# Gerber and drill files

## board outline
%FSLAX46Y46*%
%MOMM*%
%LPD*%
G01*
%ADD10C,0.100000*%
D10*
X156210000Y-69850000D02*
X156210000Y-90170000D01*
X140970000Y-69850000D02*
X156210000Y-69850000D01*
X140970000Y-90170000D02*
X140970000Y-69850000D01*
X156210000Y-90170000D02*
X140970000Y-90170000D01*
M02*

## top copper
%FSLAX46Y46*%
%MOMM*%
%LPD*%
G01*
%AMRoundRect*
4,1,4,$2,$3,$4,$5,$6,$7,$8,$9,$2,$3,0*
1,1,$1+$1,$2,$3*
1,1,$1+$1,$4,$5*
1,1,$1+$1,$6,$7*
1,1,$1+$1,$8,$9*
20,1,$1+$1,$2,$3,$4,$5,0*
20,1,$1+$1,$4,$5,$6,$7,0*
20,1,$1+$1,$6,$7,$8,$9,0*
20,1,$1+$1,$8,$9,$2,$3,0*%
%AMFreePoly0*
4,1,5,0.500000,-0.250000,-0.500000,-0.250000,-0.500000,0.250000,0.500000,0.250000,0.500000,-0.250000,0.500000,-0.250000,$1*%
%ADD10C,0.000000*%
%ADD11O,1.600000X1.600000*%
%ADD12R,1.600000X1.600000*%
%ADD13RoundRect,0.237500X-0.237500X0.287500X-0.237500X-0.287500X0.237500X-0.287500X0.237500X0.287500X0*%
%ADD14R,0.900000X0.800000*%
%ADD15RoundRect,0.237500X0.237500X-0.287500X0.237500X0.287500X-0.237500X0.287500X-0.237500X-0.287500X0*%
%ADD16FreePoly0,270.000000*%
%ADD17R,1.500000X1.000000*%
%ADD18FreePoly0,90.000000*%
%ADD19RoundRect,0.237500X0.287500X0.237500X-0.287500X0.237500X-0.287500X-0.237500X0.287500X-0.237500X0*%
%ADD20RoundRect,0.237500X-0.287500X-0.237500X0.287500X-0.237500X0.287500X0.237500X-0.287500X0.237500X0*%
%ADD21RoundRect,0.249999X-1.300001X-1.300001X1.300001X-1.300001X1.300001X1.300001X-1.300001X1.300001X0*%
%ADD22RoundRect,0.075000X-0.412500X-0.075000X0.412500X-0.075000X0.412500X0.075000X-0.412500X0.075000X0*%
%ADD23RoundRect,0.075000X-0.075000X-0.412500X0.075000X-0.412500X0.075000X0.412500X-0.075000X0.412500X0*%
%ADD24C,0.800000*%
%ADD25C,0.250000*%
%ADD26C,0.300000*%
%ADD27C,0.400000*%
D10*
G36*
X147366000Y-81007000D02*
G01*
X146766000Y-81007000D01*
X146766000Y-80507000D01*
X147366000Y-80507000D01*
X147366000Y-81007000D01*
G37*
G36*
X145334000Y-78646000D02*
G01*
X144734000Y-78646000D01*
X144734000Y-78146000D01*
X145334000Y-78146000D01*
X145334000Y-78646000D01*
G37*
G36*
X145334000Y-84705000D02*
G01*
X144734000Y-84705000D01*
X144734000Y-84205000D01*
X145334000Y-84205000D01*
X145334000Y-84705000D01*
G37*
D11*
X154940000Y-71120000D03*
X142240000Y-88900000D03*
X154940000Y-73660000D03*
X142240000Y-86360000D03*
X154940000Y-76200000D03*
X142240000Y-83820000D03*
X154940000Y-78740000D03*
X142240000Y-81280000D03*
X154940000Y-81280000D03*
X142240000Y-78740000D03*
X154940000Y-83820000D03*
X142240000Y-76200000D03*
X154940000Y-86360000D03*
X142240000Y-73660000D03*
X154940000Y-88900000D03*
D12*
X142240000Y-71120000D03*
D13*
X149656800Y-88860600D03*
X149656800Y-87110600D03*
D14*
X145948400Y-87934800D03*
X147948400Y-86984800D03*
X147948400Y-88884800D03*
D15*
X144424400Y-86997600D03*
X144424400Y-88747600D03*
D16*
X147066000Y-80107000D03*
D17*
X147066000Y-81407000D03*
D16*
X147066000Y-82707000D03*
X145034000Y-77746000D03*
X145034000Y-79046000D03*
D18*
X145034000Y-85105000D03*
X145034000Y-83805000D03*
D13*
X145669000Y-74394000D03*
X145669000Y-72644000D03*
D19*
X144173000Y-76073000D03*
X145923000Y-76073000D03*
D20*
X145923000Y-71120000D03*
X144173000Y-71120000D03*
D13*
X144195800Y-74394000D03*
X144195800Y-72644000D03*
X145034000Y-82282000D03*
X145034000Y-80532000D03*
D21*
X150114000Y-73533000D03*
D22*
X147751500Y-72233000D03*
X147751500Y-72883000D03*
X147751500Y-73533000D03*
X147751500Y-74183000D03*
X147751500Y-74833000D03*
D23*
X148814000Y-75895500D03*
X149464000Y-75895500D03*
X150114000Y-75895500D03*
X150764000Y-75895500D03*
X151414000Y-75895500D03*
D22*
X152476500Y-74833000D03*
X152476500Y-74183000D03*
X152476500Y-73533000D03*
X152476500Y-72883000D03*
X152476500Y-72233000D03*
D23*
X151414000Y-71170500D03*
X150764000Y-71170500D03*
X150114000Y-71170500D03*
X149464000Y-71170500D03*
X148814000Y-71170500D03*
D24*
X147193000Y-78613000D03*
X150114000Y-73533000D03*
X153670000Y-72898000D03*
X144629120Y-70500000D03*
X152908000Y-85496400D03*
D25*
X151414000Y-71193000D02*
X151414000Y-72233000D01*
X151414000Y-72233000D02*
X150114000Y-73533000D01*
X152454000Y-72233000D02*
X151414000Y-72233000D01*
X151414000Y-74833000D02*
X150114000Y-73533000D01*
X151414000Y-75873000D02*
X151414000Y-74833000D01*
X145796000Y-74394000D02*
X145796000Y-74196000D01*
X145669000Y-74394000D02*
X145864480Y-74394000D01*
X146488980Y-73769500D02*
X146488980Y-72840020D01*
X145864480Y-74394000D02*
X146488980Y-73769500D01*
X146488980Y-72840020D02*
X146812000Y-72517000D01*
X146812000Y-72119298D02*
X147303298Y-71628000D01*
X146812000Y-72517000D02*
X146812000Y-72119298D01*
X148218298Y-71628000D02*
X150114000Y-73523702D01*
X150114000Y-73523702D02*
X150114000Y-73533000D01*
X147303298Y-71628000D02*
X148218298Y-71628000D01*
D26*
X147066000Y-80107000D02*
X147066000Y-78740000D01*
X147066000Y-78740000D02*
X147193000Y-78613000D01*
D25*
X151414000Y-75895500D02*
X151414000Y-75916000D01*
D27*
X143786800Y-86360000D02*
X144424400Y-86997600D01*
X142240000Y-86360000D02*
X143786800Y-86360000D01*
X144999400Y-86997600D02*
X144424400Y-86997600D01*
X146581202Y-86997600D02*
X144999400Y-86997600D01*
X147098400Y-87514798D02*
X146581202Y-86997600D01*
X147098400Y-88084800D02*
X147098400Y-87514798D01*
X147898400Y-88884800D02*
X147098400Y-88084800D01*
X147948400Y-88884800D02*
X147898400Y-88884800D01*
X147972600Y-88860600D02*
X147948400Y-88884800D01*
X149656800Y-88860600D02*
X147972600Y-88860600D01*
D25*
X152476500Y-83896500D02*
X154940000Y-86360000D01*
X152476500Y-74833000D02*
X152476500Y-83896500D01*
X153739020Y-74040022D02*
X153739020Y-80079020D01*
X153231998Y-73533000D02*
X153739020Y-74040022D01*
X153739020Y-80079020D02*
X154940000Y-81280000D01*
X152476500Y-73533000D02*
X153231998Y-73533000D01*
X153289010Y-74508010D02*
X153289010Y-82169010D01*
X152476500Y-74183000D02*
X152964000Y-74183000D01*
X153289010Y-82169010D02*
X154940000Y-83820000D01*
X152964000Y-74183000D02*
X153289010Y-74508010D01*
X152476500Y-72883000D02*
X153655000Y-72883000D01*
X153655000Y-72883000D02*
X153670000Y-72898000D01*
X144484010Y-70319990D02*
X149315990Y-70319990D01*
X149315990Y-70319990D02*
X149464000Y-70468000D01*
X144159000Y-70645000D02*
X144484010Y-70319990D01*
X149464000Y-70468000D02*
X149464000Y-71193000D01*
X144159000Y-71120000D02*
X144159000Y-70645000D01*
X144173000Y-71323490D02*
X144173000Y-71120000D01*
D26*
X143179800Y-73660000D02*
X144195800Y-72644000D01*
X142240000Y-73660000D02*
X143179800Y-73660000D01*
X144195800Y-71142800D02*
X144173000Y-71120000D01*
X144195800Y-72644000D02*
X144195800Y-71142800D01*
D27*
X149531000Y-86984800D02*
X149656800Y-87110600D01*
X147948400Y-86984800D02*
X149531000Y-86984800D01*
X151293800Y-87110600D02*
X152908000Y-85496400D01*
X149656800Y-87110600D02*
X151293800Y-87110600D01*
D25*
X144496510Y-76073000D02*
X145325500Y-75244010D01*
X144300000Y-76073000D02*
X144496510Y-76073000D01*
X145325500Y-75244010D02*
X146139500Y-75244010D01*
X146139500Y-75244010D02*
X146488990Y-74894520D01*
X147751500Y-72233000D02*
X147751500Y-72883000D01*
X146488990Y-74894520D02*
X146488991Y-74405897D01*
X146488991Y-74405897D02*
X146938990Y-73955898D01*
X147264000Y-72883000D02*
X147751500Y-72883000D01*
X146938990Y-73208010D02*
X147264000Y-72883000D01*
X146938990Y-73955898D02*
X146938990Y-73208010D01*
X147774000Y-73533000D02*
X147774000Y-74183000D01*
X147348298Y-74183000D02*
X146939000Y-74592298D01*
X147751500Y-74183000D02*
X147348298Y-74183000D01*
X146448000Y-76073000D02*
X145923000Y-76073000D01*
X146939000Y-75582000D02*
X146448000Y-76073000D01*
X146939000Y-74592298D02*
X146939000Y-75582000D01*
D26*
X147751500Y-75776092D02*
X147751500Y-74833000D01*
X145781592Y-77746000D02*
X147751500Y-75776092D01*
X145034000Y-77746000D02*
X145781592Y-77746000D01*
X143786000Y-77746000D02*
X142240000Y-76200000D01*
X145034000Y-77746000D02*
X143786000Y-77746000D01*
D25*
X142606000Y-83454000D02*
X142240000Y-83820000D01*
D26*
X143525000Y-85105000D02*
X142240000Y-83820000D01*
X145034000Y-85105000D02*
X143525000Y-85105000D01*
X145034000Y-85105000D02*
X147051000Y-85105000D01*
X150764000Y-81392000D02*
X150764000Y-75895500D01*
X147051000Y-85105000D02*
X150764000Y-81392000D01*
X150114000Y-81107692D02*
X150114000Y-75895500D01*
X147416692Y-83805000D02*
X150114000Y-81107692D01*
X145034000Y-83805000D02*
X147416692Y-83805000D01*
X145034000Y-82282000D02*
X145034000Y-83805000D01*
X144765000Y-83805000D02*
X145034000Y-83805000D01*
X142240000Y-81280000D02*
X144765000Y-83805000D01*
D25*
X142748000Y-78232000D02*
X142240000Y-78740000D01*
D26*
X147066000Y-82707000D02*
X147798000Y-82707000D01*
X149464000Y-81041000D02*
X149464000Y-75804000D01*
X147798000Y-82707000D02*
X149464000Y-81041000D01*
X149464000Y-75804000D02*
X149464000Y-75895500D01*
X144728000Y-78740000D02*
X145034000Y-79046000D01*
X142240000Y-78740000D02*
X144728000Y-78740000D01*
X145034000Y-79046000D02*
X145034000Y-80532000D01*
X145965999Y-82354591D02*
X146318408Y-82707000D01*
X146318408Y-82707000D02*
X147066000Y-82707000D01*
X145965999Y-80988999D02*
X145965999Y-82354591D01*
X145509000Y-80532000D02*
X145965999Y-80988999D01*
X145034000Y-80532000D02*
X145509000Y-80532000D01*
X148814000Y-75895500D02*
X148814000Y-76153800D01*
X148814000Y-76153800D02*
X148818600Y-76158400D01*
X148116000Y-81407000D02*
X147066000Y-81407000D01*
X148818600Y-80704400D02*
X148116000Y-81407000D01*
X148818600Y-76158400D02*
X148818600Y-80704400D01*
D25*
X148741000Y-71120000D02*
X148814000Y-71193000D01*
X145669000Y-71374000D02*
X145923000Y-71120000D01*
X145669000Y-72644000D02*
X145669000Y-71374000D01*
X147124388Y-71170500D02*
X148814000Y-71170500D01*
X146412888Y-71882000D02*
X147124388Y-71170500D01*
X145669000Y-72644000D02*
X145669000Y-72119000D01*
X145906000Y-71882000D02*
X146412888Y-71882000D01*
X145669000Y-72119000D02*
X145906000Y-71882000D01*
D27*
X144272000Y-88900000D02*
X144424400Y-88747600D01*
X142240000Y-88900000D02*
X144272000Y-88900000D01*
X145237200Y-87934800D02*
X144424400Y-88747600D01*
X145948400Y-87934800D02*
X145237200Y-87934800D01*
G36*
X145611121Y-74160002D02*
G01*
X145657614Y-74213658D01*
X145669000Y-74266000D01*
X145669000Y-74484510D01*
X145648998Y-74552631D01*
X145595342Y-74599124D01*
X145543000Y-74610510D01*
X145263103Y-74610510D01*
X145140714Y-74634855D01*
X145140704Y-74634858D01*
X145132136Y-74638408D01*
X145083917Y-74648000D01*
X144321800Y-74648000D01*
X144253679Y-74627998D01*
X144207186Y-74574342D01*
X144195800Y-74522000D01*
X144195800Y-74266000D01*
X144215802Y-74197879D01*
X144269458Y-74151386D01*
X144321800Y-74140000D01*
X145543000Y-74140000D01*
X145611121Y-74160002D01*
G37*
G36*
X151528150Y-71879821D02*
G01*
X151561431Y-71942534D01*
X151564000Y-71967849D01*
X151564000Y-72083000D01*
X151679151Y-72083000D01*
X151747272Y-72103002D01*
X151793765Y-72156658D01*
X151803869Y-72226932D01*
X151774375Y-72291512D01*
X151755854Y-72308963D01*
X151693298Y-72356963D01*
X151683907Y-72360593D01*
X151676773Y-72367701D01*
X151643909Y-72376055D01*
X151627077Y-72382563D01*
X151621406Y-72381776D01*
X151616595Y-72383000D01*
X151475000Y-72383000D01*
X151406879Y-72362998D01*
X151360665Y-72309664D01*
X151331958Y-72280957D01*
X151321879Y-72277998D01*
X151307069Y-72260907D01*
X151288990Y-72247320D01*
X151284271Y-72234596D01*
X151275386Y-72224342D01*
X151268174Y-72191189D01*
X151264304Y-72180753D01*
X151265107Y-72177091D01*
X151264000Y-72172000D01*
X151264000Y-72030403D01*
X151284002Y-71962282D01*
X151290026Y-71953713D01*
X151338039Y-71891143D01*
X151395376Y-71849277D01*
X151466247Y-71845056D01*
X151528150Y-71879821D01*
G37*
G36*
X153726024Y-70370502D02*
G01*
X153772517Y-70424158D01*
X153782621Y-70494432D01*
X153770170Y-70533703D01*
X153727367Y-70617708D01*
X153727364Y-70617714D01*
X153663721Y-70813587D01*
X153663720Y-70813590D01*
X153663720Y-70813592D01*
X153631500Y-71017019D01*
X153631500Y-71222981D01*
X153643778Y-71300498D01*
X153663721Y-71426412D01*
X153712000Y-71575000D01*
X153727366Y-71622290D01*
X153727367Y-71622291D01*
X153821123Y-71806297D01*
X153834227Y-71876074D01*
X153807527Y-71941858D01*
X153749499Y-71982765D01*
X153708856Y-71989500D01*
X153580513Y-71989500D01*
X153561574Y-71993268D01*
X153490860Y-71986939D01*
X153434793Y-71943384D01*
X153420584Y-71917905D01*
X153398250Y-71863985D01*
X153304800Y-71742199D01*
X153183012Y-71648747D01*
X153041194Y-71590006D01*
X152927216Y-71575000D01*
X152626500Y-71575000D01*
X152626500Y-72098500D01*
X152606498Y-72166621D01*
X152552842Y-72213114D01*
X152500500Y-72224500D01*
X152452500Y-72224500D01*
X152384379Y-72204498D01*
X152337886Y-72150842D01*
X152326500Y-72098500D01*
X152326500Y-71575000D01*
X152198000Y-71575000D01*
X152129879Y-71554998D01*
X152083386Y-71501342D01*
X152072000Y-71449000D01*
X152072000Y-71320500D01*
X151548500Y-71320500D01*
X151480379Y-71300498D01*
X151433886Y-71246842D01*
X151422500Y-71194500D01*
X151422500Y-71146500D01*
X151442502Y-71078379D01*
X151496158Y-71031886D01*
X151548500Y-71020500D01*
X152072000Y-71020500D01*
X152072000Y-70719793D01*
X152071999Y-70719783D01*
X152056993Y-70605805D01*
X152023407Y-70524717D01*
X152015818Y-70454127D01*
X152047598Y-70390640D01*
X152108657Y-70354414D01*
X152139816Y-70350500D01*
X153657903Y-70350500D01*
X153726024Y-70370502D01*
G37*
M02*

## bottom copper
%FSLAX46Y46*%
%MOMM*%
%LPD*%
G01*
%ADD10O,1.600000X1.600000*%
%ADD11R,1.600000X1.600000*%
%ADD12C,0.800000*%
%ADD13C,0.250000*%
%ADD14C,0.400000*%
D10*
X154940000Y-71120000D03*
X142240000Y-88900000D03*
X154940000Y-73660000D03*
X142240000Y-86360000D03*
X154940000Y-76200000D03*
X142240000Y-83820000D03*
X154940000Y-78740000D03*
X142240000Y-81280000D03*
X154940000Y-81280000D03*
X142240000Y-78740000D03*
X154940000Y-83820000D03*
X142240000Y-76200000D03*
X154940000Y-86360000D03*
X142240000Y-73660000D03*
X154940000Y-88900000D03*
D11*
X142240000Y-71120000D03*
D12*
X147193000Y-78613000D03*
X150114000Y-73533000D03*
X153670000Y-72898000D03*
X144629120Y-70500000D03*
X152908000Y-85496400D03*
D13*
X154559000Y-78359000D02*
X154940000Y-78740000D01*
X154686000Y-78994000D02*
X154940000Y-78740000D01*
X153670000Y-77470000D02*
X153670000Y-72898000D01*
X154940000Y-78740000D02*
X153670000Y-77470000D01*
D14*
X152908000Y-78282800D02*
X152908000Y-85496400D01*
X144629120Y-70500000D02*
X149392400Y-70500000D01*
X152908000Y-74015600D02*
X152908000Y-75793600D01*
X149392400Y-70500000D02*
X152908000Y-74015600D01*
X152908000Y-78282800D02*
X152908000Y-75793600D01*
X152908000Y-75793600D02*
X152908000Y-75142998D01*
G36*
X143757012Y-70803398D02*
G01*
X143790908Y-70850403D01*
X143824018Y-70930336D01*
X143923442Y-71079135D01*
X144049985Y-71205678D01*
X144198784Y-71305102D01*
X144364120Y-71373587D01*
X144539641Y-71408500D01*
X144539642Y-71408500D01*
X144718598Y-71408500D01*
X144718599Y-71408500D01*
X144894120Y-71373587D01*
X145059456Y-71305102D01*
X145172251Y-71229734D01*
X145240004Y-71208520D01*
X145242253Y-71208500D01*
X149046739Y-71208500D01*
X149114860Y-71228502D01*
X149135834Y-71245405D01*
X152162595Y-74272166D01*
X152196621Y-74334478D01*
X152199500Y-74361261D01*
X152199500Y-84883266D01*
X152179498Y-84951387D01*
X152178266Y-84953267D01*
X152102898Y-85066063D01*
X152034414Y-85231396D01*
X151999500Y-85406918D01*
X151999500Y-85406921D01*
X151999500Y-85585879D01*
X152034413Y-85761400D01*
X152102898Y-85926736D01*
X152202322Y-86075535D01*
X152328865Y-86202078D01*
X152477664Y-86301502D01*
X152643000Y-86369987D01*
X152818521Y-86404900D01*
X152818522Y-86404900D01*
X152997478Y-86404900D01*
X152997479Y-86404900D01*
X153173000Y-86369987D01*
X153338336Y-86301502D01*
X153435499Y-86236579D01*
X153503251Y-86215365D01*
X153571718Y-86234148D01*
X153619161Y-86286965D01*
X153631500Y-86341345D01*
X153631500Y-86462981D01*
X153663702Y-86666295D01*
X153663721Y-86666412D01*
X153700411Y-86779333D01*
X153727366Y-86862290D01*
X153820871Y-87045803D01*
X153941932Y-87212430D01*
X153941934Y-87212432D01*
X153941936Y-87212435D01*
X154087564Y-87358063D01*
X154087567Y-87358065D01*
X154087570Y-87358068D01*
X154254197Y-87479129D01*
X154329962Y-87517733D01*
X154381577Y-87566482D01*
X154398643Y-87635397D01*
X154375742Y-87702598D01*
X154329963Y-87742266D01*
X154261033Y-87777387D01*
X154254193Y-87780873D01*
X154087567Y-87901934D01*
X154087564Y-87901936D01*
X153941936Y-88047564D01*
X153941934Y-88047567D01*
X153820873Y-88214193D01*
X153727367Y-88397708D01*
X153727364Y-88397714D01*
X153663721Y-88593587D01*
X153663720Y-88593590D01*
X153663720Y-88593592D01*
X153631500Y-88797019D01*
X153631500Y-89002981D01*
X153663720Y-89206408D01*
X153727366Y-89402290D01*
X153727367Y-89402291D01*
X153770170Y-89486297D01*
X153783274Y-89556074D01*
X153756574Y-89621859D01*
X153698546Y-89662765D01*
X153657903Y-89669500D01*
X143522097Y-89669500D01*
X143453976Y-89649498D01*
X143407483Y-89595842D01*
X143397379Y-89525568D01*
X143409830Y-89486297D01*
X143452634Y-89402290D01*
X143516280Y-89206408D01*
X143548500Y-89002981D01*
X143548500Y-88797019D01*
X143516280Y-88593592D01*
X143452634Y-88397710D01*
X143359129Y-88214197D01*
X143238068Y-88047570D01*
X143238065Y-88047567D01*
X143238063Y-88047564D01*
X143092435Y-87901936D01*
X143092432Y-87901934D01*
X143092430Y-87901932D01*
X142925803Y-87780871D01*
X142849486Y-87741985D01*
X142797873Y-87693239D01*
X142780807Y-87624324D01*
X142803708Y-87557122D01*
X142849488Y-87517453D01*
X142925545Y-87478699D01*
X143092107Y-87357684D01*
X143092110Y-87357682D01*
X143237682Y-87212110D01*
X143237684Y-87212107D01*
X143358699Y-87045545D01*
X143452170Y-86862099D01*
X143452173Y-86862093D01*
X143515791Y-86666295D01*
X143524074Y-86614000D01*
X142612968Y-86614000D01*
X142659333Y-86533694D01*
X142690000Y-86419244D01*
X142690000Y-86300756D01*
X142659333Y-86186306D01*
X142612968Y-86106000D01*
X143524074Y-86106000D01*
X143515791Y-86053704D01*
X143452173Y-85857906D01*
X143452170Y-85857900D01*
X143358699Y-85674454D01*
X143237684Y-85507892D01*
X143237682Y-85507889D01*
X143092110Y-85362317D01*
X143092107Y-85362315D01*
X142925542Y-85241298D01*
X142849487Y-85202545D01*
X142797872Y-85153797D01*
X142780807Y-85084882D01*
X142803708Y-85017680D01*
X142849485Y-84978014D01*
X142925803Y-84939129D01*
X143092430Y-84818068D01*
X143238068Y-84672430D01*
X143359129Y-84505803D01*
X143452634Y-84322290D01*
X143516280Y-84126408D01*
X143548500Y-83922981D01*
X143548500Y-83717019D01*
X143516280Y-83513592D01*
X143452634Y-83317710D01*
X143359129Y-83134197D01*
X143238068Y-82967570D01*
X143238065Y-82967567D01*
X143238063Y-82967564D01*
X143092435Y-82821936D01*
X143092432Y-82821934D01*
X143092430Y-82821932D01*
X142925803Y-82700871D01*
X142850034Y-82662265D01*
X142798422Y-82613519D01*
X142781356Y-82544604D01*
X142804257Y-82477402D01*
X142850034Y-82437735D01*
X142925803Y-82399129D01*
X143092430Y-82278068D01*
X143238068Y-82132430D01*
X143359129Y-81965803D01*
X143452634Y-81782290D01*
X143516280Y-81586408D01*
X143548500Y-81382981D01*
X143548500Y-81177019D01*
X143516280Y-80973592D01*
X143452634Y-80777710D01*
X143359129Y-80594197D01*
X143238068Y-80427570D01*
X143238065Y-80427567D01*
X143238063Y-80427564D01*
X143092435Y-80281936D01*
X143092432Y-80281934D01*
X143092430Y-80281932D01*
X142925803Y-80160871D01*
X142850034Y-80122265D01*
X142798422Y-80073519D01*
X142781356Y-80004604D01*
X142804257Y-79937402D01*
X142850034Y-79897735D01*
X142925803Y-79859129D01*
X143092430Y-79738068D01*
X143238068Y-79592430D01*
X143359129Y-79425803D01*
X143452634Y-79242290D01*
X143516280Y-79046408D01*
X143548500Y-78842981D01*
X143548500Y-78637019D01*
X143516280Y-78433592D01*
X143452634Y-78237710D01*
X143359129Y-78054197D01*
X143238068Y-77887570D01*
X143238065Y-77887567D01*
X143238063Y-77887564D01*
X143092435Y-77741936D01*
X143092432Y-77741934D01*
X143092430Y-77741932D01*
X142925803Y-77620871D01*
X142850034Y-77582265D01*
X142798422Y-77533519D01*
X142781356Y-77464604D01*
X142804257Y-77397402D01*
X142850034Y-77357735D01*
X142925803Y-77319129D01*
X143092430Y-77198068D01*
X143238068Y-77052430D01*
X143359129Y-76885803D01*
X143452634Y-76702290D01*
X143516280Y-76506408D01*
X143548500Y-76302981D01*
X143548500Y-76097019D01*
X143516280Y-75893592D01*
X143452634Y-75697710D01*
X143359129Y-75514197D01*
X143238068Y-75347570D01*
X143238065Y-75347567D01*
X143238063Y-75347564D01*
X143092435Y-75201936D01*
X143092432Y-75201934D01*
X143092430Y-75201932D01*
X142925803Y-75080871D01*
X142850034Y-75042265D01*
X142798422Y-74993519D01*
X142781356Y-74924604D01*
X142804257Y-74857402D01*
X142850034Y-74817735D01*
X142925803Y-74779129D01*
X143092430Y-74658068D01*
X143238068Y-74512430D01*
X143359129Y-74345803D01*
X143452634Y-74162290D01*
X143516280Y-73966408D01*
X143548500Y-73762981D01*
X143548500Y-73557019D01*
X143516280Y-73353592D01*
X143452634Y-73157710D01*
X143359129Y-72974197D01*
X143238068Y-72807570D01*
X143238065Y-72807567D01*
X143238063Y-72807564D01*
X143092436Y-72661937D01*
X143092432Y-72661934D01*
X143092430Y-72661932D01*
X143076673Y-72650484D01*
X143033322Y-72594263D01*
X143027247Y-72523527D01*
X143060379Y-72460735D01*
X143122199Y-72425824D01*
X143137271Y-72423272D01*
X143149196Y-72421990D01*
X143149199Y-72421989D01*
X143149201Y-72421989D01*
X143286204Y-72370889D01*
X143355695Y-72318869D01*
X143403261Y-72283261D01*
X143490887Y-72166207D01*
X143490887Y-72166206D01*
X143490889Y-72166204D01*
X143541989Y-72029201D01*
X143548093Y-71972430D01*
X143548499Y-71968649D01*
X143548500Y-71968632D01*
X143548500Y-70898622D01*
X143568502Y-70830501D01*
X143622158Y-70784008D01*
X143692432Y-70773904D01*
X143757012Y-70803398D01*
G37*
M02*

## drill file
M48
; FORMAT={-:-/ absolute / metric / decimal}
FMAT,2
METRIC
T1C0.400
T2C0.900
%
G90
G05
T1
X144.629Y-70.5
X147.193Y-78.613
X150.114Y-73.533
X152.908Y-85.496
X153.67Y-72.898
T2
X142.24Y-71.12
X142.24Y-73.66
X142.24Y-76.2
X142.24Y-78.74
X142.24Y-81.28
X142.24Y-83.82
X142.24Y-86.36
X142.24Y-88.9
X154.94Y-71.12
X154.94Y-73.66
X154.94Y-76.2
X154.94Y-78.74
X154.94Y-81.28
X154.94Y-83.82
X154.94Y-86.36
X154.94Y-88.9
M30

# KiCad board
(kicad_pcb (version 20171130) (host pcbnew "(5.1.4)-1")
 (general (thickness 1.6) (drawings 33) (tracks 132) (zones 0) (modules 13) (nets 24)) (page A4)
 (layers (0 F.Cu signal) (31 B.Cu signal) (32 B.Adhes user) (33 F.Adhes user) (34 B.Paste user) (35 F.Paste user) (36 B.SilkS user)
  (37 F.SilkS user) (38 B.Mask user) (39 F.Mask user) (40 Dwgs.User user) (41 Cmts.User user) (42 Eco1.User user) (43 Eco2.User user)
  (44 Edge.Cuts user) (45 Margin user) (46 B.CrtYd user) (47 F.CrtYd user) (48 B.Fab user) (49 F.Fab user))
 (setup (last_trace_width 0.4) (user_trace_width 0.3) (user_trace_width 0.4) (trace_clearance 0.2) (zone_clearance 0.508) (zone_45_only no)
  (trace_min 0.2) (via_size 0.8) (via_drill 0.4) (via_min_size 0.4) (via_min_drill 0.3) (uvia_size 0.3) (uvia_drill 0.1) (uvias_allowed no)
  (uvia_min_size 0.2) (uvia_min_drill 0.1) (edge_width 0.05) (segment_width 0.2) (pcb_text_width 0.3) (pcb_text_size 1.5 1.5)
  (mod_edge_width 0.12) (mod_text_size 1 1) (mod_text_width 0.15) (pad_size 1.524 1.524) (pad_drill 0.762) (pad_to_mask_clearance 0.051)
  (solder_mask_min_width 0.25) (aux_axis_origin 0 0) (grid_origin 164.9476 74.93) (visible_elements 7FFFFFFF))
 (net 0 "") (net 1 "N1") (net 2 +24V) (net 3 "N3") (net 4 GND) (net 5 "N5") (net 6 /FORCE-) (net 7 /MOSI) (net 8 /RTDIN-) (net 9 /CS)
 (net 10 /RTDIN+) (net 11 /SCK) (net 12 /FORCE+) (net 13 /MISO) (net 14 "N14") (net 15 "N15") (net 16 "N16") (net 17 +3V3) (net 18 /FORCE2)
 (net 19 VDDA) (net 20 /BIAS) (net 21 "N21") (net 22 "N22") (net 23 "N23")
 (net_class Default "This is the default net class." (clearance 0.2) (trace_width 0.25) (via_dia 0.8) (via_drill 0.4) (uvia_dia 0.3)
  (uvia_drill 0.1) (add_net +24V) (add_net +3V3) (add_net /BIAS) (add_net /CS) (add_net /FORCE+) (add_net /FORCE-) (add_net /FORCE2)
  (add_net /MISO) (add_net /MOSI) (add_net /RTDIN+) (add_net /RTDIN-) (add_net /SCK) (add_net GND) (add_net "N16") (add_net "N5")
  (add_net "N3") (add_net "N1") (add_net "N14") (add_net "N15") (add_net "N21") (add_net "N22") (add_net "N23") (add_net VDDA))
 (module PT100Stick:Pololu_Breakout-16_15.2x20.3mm (layer F.Cu) (at 142.24 71.12)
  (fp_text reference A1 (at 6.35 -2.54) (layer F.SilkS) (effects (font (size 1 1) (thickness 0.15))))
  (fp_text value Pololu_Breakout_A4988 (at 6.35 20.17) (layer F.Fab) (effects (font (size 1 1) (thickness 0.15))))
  (pad 16 thru_hole oval (at 12.7 0) (size 1.6 1.6) (drill 0.9) (layers *.Cu *.Mask) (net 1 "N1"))
  (pad 8 thru_hole oval (at 0 17.78) (size 1.6 1.6) (drill 0.9) (layers *.Cu *.Mask) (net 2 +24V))
  (pad 15 thru_hole oval (at 12.7 2.54) (size 1.6 1.6) (drill 0.9) (layers *.Cu *.Mask) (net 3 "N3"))
  (pad 7 thru_hole oval (at 0 15.24) (size 1.6 1.6) (drill 0.9) (layers *.Cu *.Mask) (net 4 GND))
  (pad 14 thru_hole oval (at 12.7 5.08) (size 1.6 1.6) (drill 0.9) (layers *.Cu *.Mask) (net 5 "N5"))
  (pad 6 thru_hole oval (at 0 12.7) (size 1.6 1.6) (drill 0.9) (layers *.Cu *.Mask) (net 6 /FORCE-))
  (pad 13 thru_hole oval (at 12.7 7.62) (size 1.6 1.6) (drill 0.9) (layers *.Cu *.Mask) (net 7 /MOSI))
  (pad 5 thru_hole oval (at 0 10.16) (size 1.6 1.6) (drill 0.9) (layers *.Cu *.Mask) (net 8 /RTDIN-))
  (pad 12 thru_hole oval (at 12.7 10.16) (size 1.6 1.6) (drill 0.9) (layers *.Cu *.Mask) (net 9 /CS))
  (pad 4 thru_hole oval (at 0 7.62) (size 1.6 1.6) (drill 0.9) (layers *.Cu *.Mask) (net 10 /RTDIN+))
  (pad 11 thru_hole oval (at 12.7 12.7) (size 1.6 1.6) (drill 0.9) (layers *.Cu *.Mask) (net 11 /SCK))
  (pad 3 thru_hole oval (at 0 5.08) (size 1.6 1.6) (drill 0.9) (layers *.Cu *.Mask) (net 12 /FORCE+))
  (pad 10 thru_hole oval (at 12.7 15.24) (size 1.6 1.6) (drill 0.9) (layers *.Cu *.Mask) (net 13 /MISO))
  (pad 2 thru_hole oval (at 0 2.54) (size 1.6 1.6) (drill 0.9) (layers *.Cu *.Mask) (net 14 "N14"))
  (pad 9 thru_hole oval (at 12.7 17.78) (size 1.6 1.6) (drill 0.9) (layers *.Cu *.Mask) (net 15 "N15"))
  (pad 1 thru_hole rect (at 0 0) (size 1.6 1.6) (drill 0.9) (layers *.Cu *.Mask) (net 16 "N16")))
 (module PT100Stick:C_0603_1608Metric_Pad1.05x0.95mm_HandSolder (layer F.Cu) (at 149.6568 87.9856 270)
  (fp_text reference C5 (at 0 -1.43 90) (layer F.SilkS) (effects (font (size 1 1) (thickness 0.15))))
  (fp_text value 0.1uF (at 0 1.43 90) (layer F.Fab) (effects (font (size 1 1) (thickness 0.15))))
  (pad 2 smd roundrect (at 0.875 0 270) (size 1.05 0.95) (layers F.Cu F.Paste F.Mask) (roundrect_rratio 0.25) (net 4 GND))
  (pad 1 smd roundrect (at -0.875 0 270) (size 1.05 0.95) (layers F.Cu F.Paste F.Mask) (roundrect_rratio 0.25) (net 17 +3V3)))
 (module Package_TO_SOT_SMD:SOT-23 (layer F.Cu) (at 146.9484 87.9348 180)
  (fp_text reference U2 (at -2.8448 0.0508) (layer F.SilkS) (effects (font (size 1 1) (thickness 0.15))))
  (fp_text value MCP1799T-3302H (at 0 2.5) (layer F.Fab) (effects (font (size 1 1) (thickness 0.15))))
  (pad 3 smd rect (at 1 0 180) (size 0.9 0.8) (layers F.Cu F.Paste F.Mask) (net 2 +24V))
  (pad 2 smd rect (at -1 0.95 180) (size 0.9 0.8) (layers F.Cu F.Paste F.Mask) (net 17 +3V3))
  (pad 1 smd rect (at -1 -0.95 180) (size 0.9 0.8) (layers F.Cu F.Paste F.Mask) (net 4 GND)))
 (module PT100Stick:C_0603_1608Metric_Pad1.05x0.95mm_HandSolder (layer F.Cu) (at 144.4244 87.8726 90)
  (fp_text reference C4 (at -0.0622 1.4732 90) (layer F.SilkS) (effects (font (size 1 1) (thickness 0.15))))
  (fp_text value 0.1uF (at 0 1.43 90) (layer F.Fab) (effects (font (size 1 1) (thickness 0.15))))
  (pad 2 smd roundrect (at 0.875 0 90) (size 1.05 0.95) (layers F.Cu F.Paste F.Mask) (roundrect_rratio 0.25) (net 4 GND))
  (pad 1 smd roundrect (at -0.875 0 90) (size 1.05 0.95) (layers F.Cu F.Paste F.Mask) (roundrect_rratio 0.25) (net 2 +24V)))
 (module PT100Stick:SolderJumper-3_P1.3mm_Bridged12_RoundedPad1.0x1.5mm (layer F.Cu) (at 147.066 81.407 270)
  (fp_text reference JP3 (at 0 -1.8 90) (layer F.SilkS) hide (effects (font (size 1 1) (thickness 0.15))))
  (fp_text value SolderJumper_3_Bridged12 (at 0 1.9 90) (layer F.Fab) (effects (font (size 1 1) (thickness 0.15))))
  (fp_poly (pts (xy -0.9 -0.3) (xy -0.4 -0.3) (xy -0.4 0.3) (xy -0.9 0.3)) (layer F.Cu) (width 0))
  (pad 1 smd custom (at -1.3 0 270) (size 1 0.5) (layers F.Cu F.Mask) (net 4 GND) (zone_connect 2)
   (options (clearance outline) (anchor rect)) (primitives))
  (pad 2 smd rect (at 0 0 270) (size 1 1.5) (layers F.Cu F.Mask) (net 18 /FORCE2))
  (pad 3 smd custom (at 1.3 0 270) (size 1 0.5) (layers F.Cu F.Mask) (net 10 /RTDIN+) (zone_connect 2)
   (options (clearance outline) (anchor rect)) (primitives)))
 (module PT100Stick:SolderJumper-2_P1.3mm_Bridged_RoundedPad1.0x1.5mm (layer F.Cu) (at 145.034 78.396 270)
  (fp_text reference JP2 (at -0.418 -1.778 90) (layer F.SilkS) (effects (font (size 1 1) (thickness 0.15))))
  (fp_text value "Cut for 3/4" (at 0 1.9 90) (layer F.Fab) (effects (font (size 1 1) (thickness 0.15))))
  (fp_poly (pts (xy 0.25 -0.3) (xy -0.25 -0.3) (xy -0.25 0.3) (xy 0.25 0.3)) (layer F.Cu) (width 0))
  (pad 1 smd custom (at -0.65 0 270) (size 1 0.5) (layers F.Cu F.Mask) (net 12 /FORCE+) (zone_connect 2)
   (options (clearance outline) (anchor rect)) (primitives))
  (pad 2 smd custom (at 0.65 0 270) (size 1 0.5) (layers F.Cu F.Mask) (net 10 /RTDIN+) (zone_connect 2)
   (options (clearance outline) (anchor rect)) (primitives)))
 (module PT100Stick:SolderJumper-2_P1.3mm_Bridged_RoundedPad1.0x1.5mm (layer F.Cu) (at 145.034 84.455 90)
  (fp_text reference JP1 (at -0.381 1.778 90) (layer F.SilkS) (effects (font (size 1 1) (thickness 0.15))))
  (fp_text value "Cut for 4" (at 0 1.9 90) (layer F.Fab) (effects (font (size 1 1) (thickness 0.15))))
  (fp_poly (pts (xy 0.25 -0.3) (xy -0.25 -0.3) (xy -0.25 0.3) (xy 0.25 0.3)) (layer F.Cu) (width 0))
  (pad 1 smd custom (at -0.65 0 90) (size 1 0.5) (layers F.Cu F.Mask) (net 6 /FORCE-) (zone_connect 2)
   (options (clearance outline) (anchor rect)) (primitives))
  (pad 2 smd custom (at 0.65 0 90) (size 1 0.5) (layers F.Cu F.Mask) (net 8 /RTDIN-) (zone_connect 2)
   (options (clearance outline) (anchor rect)) (primitives)))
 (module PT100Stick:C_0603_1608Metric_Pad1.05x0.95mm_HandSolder (layer F.Cu) (at 145.669 73.519 270)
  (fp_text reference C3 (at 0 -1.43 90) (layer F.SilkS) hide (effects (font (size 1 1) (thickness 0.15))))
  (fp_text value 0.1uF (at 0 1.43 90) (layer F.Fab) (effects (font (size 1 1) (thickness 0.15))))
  (pad 2 smd roundrect (at 0.875 0 270) (size 1.05 0.95) (layers F.Cu F.Paste F.Mask) (roundrect_rratio 0.25) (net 4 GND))
  (pad 1 smd roundrect (at -0.875 0 270) (size 1.05 0.95) (layers F.Cu F.Paste F.Mask) (roundrect_rratio 0.25) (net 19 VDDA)))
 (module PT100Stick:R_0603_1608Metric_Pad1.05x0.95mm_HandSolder (layer F.Cu) (at 145.048 76.073 180)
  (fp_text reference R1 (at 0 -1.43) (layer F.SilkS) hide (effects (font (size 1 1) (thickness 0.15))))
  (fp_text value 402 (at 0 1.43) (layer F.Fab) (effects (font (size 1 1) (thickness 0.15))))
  (pad 2 smd roundrect (at 0.875 0 180) (size 1.05 0.95) (layers F.Cu F.Paste F.Mask) (roundrect_rratio 0.25) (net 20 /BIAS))
  (pad 1 smd roundrect (at -0.875 0 180) (size 1.05 0.95) (layers F.Cu F.Paste F.Mask) (roundrect_rratio 0.25) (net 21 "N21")))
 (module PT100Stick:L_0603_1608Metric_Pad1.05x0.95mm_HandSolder (layer F.Cu) (at 145.048 71.12)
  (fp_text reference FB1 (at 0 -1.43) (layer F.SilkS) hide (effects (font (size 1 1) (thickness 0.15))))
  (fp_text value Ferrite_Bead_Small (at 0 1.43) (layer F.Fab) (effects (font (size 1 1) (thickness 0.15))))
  (pad 2 smd roundrect (at 0.875 0) (size 1.05 0.95) (layers F.Cu F.Paste F.Mask) (roundrect_rratio 0.25) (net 19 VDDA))
  (pad 1 smd roundrect (at -0.875 0) (size 1.05 0.95) (layers F.Cu F.Paste F.Mask) (roundrect_rratio 0.25) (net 17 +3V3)))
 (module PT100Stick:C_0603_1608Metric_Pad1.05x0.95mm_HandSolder (layer F.Cu) (at 144.1958 73.519 270)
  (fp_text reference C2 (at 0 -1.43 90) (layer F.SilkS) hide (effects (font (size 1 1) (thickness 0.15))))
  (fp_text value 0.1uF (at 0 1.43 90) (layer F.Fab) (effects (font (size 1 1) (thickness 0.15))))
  (pad 2 smd roundrect (at 0.875 0 270) (size 1.05 0.95) (layers F.Cu F.Paste F.Mask) (roundrect_rratio 0.25) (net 4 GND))
  (pad 1 smd roundrect (at -0.875 0 270) (size 1.05 0.95) (layers F.Cu F.Paste F.Mask) (roundrect_rratio 0.25) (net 17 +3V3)))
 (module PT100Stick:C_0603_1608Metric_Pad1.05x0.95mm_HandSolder (layer F.Cu) (at 145.034 81.407 270)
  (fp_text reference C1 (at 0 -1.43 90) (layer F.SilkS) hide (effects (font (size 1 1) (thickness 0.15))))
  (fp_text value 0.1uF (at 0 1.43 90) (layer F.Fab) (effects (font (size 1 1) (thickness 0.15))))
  (pad 2 smd roundrect (at 0.875 0 270) (size 1.05 0.95) (layers F.Cu F.Paste F.Mask) (roundrect_rratio 0.25) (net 8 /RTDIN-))
  (pad 1 smd roundrect (at -0.875 0 270) (size 1.05 0.95) (layers F.Cu F.Paste F.Mask) (roundrect_rratio 0.25) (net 10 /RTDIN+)))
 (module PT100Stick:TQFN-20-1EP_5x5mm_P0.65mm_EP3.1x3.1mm (layer F.Cu) (at 150.114 73.533)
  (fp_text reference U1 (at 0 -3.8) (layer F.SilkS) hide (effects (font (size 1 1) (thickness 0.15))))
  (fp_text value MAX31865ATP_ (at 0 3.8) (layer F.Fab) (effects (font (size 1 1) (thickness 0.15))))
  (pad 21 smd roundrect (at 0 0) (size 3.1 3.1) (layers F.Cu F.Mask) (roundrect_rratio 0.08064499999999999) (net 4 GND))
  (pad "" smd roundrect (at -0.775 -0.775) (size 1.25 1.25) (layers F.Paste) (roundrect_rratio 0.2))
  (pad "" smd roundrect (at -0.775 0.775) (size 1.25 1.25) (layers F.Paste) (roundrect_rratio 0.2))
  (pad "" smd roundrect (at 0.775 -0.775) (size 1.25 1.25) (layers F.Paste) (roundrect_rratio 0.2))
  (pad "" smd roundrect (at 0.775 0.775) (size 1.25 1.25) (layers F.Paste) (roundrect_rratio 0.2))
  (pad 1 smd roundrect (at -2.3625 -1.3) (size 0.975 0.3) (layers F.Cu F.Paste F.Mask) (roundrect_rratio 0.25) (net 20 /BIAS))
  (pad 2 smd roundrect (at -2.3625 -0.65) (size 0.975 0.3) (layers F.Cu F.Paste F.Mask) (roundrect_rratio 0.25) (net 20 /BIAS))
  (pad 3 smd roundrect (at -2.3625 0) (size 0.975 0.3) (layers F.Cu F.Paste F.Mask) (roundrect_rratio 0.25) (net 21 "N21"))
  (pad 4 smd roundrect (at -2.3625 0.65) (size 0.975 0.3) (layers F.Cu F.Paste F.Mask) (roundrect_rratio 0.25) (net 21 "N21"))
  (pad 5 smd roundrect (at -2.3625 1.3) (size 0.975 0.3) (layers F.Cu F.Paste F.Mask) (roundrect_rratio 0.25) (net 12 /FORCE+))
  (pad 6 smd roundrect (at -1.3 2.3625) (size 0.3 0.975) (layers F.Cu F.Paste F.Mask) (roundrect_rratio 0.25) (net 18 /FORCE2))
  (pad 7 smd roundrect (at -0.65 2.3625) (size 0.3 0.975) (layers F.Cu F.Paste F.Mask) (roundrect_rratio 0.25) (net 10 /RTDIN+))
  (pad 8 smd roundrect (at 0 2.3625) (size 0.3 0.975) (layers F.Cu F.Paste F.Mask) (roundrect_rratio 0.25) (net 8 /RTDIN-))
  (pad 9 smd roundrect (at 0.65 2.3625) (size 0.3 0.975) (layers F.Cu F.Paste F.Mask) (roundrect_rratio 0.25) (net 6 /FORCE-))
  (pad 10 smd roundrect (at 1.3 2.3625) (size 0.3 0.975) (layers F.Cu F.Paste F.Mask) (roundrect_rratio 0.25) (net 4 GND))
  (pad 11 smd roundrect (at 2.3625 1.3) (size 0.975 0.3) (layers F.Cu F.Paste F.Mask) (roundrect_rratio 0.25) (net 13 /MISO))
  (pad 12 smd roundrect (at 2.3625 0.65) (size 0.975 0.3) (layers F.Cu F.Paste F.Mask) (roundrect_rratio 0.25) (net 11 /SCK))
  (pad 13 smd roundrect (at 2.3625 0) (size 0.975 0.3) (layers F.Cu F.Paste F.Mask) (roundrect_rratio 0.25) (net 9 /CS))
  (pad 14 smd roundrect (at 2.3625 -0.65) (size 0.975 0.3) (layers F.Cu F.Paste F.Mask) (roundrect_rratio 0.25) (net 7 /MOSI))
  (pad 15 smd roundrect (at 2.3625 -1.3) (size 0.975 0.3) (layers F.Cu F.Paste F.Mask) (roundrect_rratio 0.25) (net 4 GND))
  (pad 16 smd roundrect (at 1.3 -2.3625) (size 0.3 0.975) (layers F.Cu F.Paste F.Mask) (roundrect_rratio 0.25) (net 4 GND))
  (pad 17 smd roundrect (at 0.65 -2.3625) (size 0.3 0.975) (layers F.Cu F.Paste F.Mask) (roundrect_rratio 0.25) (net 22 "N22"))
  (pad 18 smd roundrect (at 0 -2.3625) (size 0.3 0.975) (layers F.Cu F.Paste F.Mask) (roundrect_rratio 0.25) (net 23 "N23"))
  (pad 19 smd roundrect (at -0.65 -2.3625) (size 0.3 0.975) (layers F.Cu F.Paste F.Mask) (roundrect_rratio 0.25) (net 17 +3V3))
  (pad 20 smd roundrect (at -1.3 -2.3625) (size 0.3 0.975) (layers F.Cu F.Paste F.Mask) (roundrect_rratio 0.25) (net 19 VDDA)))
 (gr_line (start 156.21 69.85) (end 156.21 90.17) (layer Edge.Cuts) (width 0.1))
 (gr_line (start 140.97 69.85) (end 156.21 69.85) (layer Edge.Cuts) (width 0.1))
 (gr_line (start 140.97 90.17) (end 140.97 69.85) (layer Edge.Cuts) (width 0.1))
 (gr_line (start 156.21 90.17) (end 140.97 90.17) (layer Edge.Cuts) (width 0.1))
 (segment (start 151.414 71.193) (end 151.414 72.233) (width 0.25) (layer F.Cu) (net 4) (status 30))
 (segment (start 151.414 72.233) (end 150.114 73.533) (width 0.25) (layer F.Cu) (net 4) (status 30))
 (segment (start 152.454 72.233) (end 151.414 72.233) (width 0.25) (layer F.Cu) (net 4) (status 30))
 (segment (start 151.414 74.833) (end 150.114 73.533) (width 0.25) (layer F.Cu) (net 4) (status 30))
 (segment (start 151.414 75.873) (end 151.414 74.833) (width 0.25) (layer F.Cu) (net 4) (status 30))
 (segment (start 145.796 74.394) (end 145.796 74.196) (width 0.25) (layer F.Cu) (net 4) (status 30))
 (segment (start 145.669 74.394) (end 145.86448 74.394) (width 0.25) (layer F.Cu) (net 4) (status 30))
 (segment (start 146.48898 73.7695) (end 146.48898 72.84002) (width 0.25) (layer F.Cu) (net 4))
 (segment (start 145.86448 74.394) (end 146.48898 73.7695) (width 0.25) (layer F.Cu) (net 4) (status 10))
 (segment (start 146.48898 72.84002) (end 146.812 72.517) (width 0.25) (layer F.Cu) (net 4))
 (segment (start 146.812 72.119298) (end 147.303298 71.628) (width 0.25) (layer F.Cu) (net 4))
 (segment (start 146.812 72.517) (end 146.812 72.119298) (width 0.25) (layer F.Cu) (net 4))
 (segment (start 148.218298 71.628) (end 150.114 73.523702) (width 0.25) (layer F.Cu) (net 4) (status 20))
 (segment (start 150.114 73.523702) (end 150.114 73.533) (width 0.25) (layer F.Cu) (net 4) (status 30))
 (segment (start 147.303298 71.628) (end 148.218298 71.628) (width 0.25) (layer F.Cu) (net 4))
 (via (at 147.193 78.613) (size 0.8) (drill 0.4) (layers F.Cu B.Cu) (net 4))
 (segment (start 147.066 80.107) (end 147.066 78.74) (width 0.3) (layer F.Cu) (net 4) (status 10))
 (segment (start 147.066 78.74) (end 147.193 78.613) (width 0.3) (layer F.Cu) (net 4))
 (segment (start 151.414 75.8955) (end 151.414 75.916) (width 0.25) (layer F.Cu) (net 4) (status 30))
 (via (at 150.114 73.533) (size 0.8) (drill 0.4) (layers F.Cu B.Cu) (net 4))
 (segment (start 143.7868 86.36) (end 144.4244 86.9976) (width 0.4) (layer F.Cu) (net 4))
 (segment (start 142.24 86.36) (end 143.7868 86.36) (width 0.4) (layer F.Cu) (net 4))
 (segment (start 144.9994 86.9976) (end 144.4244 86.9976) (width 0.4) (layer F.Cu) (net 4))
 (segment (start 146.581202 86.9976) (end 144.9994 86.9976) (width 0.4) (layer F.Cu) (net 4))
 (segment (start 147.0984 87.514798) (end 146.581202 86.9976) (width 0.4) (layer F.Cu) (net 4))
 (segment (start 147.0984 88.0848) (end 147.0984 87.514798) (width 0.4) (layer F.Cu) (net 4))
 (segment (start 147.8984 88.8848) (end 147.0984 88.0848) (width 0.4) (layer F.Cu) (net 4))
 (segment (start 147.9484 88.8848) (end 147.8984 88.8848) (width 0.4) (layer F.Cu) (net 4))
 (segment (start 147.9726 88.8606) (end 147.9484 88.8848) (width 0.4) (layer F.Cu) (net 4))
 (segment (start 149.6568 88.8606) (end 147.9726 88.8606) (width 0.4) (layer F.Cu) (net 4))
 (segment (start 152.4765 83.8965) (end 154.94 86.36) (width 0.25) (layer F.Cu) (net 13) (status 20))
 (segment (start 152.4765 74.833) (end 152.4765 83.8965) (width 0.25) (layer F.Cu) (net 13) (status 10))
 (segment (start 153.73902 74.040022) (end 153.73902 80.07902) (width 0.25) (layer F.Cu) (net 9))
 (segment (start 153.231998 73.533) (end 153.73902 74.040022) (width 0.25) (layer F.Cu) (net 9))
 (segment (start 153.73902 80.07902) (end 154.94 81.28) (width 0.25) (layer F.Cu) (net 9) (status 20))
 (segment (start 152.4765 73.533) (end 153.231998 73.533) (width 0.25) (layer F.Cu) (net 9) (status 10))
 (segment (start 153.28901 74.50801) (end 153.28901 82.16901) (width 0.25) (layer F.Cu) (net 11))
 (segment (start 152.4765 74.183) (end 152.964 74.183) (width 0.25) (layer F.Cu) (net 11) (status 10))
 (segment (start 153.28901 82.16901) (end 154.94 83.82) (width 0.25) (layer F.Cu) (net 11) (status 20))
 (segment (start 152.964 74.183) (end 153.28901 74.50801) (width 0.25) (layer F.Cu) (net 11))
 (segment (start 154.559 78.359) (end 154.94 78.74) (width 0.25) (layer B.Cu) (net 7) (status 30))
 (segment (start 154.686 78.994) (end 154.94 78.74) (width 0.25) (layer B.Cu) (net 7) (status 30))
 (via (at 153.67 72.898) (size 0.8) (drill 0.4) (layers F.Cu B.Cu) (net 7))
 (segment (start 152.4765 72.883) (end 153.655 72.883) (width 0.25) (layer F.Cu) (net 7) (status 10))
 (segment (start 153.655 72.883) (end 153.67 72.898) (width 0.25) (layer F.Cu) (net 7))
 (segment (start 153.67 77.47) (end 153.67 72.898) (width 0.25) (layer B.Cu) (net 7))
 (segment (start 154.94 78.74) (end 153.67 77.47) (width 0.25) (layer B.Cu) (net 7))
 (segment (start 144.48401 70.31999) (end 149.31599 70.31999) (width 0.25) (layer F.Cu) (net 17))
 (segment (start 149.31599 70.31999) (end 149.464 70.468) (width 0.25) (layer F.Cu) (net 17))
 (segment (start 144.159 70.645) (end 144.48401 70.31999) (width 0.25) (layer F.Cu) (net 17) (status 10))
 (segment (start 149.464 70.468) (end 149.464 71.193) (width 0.25) (layer F.Cu) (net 17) (status 20))
 (segment (start 144.159 71.12) (end 144.159 70.645) (width 0.25) (layer F.Cu) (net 17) (status 30))
 (segment (start 144.173 71.32349) (end 144.173 71.12) (width 0.25) (layer F.Cu) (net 17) (status 30))
 (segment (start 143.1798 73.66) (end 144.1958 72.644) (width 0.3) (layer F.Cu) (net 17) (status 20))
 (segment (start 142.24 73.66) (end 143.1798 73.66) (width 0.3) (layer F.Cu) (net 17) (status 10))
 (segment (start 144.1958 71.1428) (end 144.173 71.12) (width 0.3) (layer F.Cu) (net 17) (status 30))
 (segment (start 144.1958 72.644) (end 144.1958 71.1428) (width 0.3) (layer F.Cu) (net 17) (status 30))
 (via (at 144.62912 70.5) (size 0.8) (drill 0.4) (layers F.Cu B.Cu) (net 17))
 (segment (start 149.531 86.9848) (end 149.6568 87.1106) (width 0.4) (layer F.Cu) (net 17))
 (segment (start 147.9484 86.9848) (end 149.531 86.9848) (width 0.4) (layer F.Cu) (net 17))
 (via (at 152.908 85.4964) (size 0.8) (drill 0.4) (layers F.Cu B.Cu) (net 17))
 (segment (start 151.2938 87.1106) (end 152.908 85.4964) (width 0.4) (layer F.Cu) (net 17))
 (segment (start 149.6568 87.1106) (end 151.2938 87.1106) (width 0.4) (layer F.Cu) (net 17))
 (segment (start 152.908 78.2828) (end 152.908 85.4964) (width 0.4) (layer B.Cu) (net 17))
 (segment (start 144.62912 70.5) (end 149.3924 70.5) (width 0.4) (layer B.Cu) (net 17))
 (segment (start 152.908 74.0156) (end 152.908 75.7936) (width 0.4) (layer B.Cu) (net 17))
 (segment (start 149.3924 70.5) (end 152.908 74.0156) (width 0.4) (layer B.Cu) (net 17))
 (segment (start 152.908 78.2828) (end 152.908 75.7936) (width 0.4) (layer B.Cu) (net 17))
 (segment (start 152.908 75.7936) (end 152.908 75.142998) (width 0.4) (layer B.Cu) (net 17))
 (segment (start 144.49651 76.073) (end 145.3255 75.24401) (width 0.25) (layer F.Cu) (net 20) (status 10))
 (segment (start 144.3 76.073) (end 144.49651 76.073) (width 0.25) (layer F.Cu) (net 20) (status 30))
 (segment (start 145.3255 75.24401) (end 146.1395 75.24401) (width 0.25) (layer F.Cu) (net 20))
 (segment (start 146.1395 75.24401) (end 146.48899 74.89452) (width 0.25) (layer F.Cu) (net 20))
 (segment (start 147.7515 72.233) (end 147.7515 72.883) (width 0.25) (layer F.Cu) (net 20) (status 30))
 (segment (start 146.48899 74.89452) (end 146.488991 74.405897) (width 0.25) (layer F.Cu) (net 20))
 (segment (start 146.488991 74.405897) (end 146.93899 73.955898) (width 0.25) (layer F.Cu) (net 20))
 (segment (start 147.264 72.883) (end 147.7515 72.883) (width 0.25) (layer F.Cu) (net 20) (status 30))
 (segment (start 146.93899 73.20801) (end 147.264 72.883) (width 0.25) (layer F.Cu) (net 20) (status 20))
 (segment (start 146.93899 73.955898) (end 146.93899 73.20801) (width 0.25) (layer F.Cu) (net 20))
 (segment (start 147.774 73.533) (end 147.774 74.183) (width 0.25) (layer F.Cu) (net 21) (status 30))
 (segment (start 147.348298 74.183) (end 146.939 74.592298) (width 0.25) (layer F.Cu) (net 21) (status 10))
 (segment (start 147.7515 74.183) (end 147.348298 74.183) (width 0.25) (layer F.Cu) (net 21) (status 30))
 (segment (start 146.448 76.073) (end 145.923 76.073) (width 0.25) (layer F.Cu) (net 21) (status 20))
 (segment (start 146.939 75.582) (end 146.448 76.073) (width 0.25) (layer F.Cu) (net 21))
 (segment (start 146.939 74.592298) (end 146.939 75.582) (width 0.25) (layer F.Cu) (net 21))
 (segment (start 147.7515 75.776092) (end 147.7515 74.833) (width 0.3) (layer F.Cu) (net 12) (status 20))
 (segment (start 145.781592 77.746) (end 147.7515 75.776092) (width 0.3) (layer F.Cu) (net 12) (status 10))
 (segment (start 145.034 77.746) (end 145.781592 77.746) (width 0.3) (layer F.Cu) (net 12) (status 30))
 (segment (start 143.786 77.746) (end 142.24 76.2) (width 0.3) (layer F.Cu) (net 12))
 (segment (start 145.034 77.746) (end 143.786 77.746) (width 0.3) (layer F.Cu) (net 12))
 (segment (start 142.606 83.454) (end 142.24 83.82) (width 0.25) (layer F.Cu) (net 6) (status 30))
 (segment (start 143.525 85.105) (end 142.24 83.82) (width 0.3) (layer F.Cu) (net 6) (status 20))
 (segment (start 145.034 85.105) (end 143.525 85.105) (width 0.3) (layer F.Cu) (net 6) (status 10))
 (segment (start 145.034 85.105) (end 147.051 85.105) (width 0.3) (layer F.Cu) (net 6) (status 10))
 (segment (start 150.764 81.392) (end 150.764 75.8955) (width 0.3) (layer F.Cu) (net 6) (status 20))
 (segment (start 147.051 85.105) (end 150.764 81.392) (width 0.3) (layer F.Cu) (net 6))
 (segment (start 150.114 81.107692) (end 150.114 75.8955) (width 0.3) (layer F.Cu) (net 8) (status 20))
 (segment (start 147.416692 83.805) (end 150.114 81.107692) (width 0.3) (layer F.Cu) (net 8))
 (segment (start 145.034 83.805) (end 147.416692 83.805) (width 0.3) (layer F.Cu) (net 8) (status 10))
 (segment (start 145.034 82.282) (end 145.034 83.805) (width 0.3) (layer F.Cu) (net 8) (status 30))
 (segment (start 144.765 83.805) (end 145.034 83.805) (width 0.3) (layer F.Cu) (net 8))
 (segment (start 142.24 81.28) (end 144.765 83.805) (width 0.3) (layer F.Cu) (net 8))
 (segment (start 142.748 78.232) (end 142.24 78.74) (width 0.25) (layer F.Cu) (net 10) (status 30))
 (segment (start 147.066 82.707) (end 147.798 82.707) (width 0.3) (layer F.Cu) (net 10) (status 30))
 (segment (start 149.464 81.041) (end 149.464 75.804) (width 0.3) (layer F.Cu) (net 10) (status 20))
 (segment (start 147.798 82.707) (end 149.464 81.041) (width 0.3) (layer F.Cu) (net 10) (status 10))
 (segment (start 149.464 75.804) (end 149.464 75.8955) (width 0.3) (layer F.Cu) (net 10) (status 30))
 (segment (start 144.728 78.74) (end 145.034 79.046) (width 0.3) (layer F.Cu) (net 10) (status 30))
 (segment (start 142.24 78.74) (end 144.728 78.74) (width 0.3) (layer F.Cu) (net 10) (status 30))
 (segment (start 145.034 79.046) (end 145.034 80.532) (width 0.3) (layer F.Cu) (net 10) (status 30))
 (segment (start 145.965999 82.354591) (end 146.318408 82.707) (width 0.3) (layer F.Cu) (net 10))
 (segment (start 146.318408 82.707) (end 147.066 82.707) (width 0.3) (layer F.Cu) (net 10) (status 20))
 (segment (start 145.965999 80.988999) (end 145.965999 82.354591) (width 0.3) (layer F.Cu) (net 10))
 (segment (start 145.509 80.532) (end 145.965999 80.988999) (width 0.3) (layer F.Cu) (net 10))
 (segment (start 145.034 80.532) (end 145.509 80.532) (width 0.3) (layer F.Cu) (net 10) (status 10))
 (segment (start 148.814 75.8955) (end 148.814 76.1538) (width 0.3) (layer F.Cu) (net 18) (status 30))
 (segment (start 148.814 76.1538) (end 148.8186 76.1584) (width 0.3) (layer F.Cu) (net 18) (status 30))
 (segment (start 148.116 81.407) (end 147.066 81.407) (width 0.3) (layer F.Cu) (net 18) (status 20))
 (segment (start 148.8186 80.7044) (end 148.116 81.407) (width 0.3) (layer F.Cu) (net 18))
 (segment (start 148.8186 76.1584) (end 148.8186 80.7044) (width 0.3) (layer F.Cu) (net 18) (status 10))
 (segment (start 148.741 71.12) (end 148.814 71.193) (width 0.25) (layer F.Cu) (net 19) (status 30))
 (segment (start 145.669 71.374) (end 145.923 71.12) (width 0.25) (layer F.Cu) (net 19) (status 30))
 (segment (start 145.669 72.644) (end 145.669 71.374) (width 0.25) (layer F.Cu) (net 19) (status 30))
 (segment (start 147.124388 71.1705) (end 148.814 71.1705) (width 0.25) (layer F.Cu) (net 19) (status 20))
 (segment (start 146.412888 71.882) (end 147.124388 71.1705) (width 0.25) (layer F.Cu) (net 19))
 (segment (start 145.669 72.644) (end 145.669 72.119) (width 0.25) (layer F.Cu) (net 19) (status 30))
 (segment (start 145.906 71.882) (end 146.412888 71.882) (width 0.25) (layer F.Cu) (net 19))
 (segment (start 145.669 72.119) (end 145.906 71.882) (width 0.25) (layer F.Cu) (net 19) (status 10))
 (segment (start 144.272 88.9) (end 144.4244 88.7476) (width 0.4) (layer F.Cu) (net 2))
 (segment (start 142.24 88.9) (end 144.272 88.9) (width 0.4) (layer F.Cu) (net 2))
 (segment (start 145.2372 87.9348) (end 144.4244 88.7476) (width 0.4) (layer F.Cu) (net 2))
 (segment (start 145.9484 87.9348) (end 145.2372 87.9348) (width 0.4) (layer F.Cu) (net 2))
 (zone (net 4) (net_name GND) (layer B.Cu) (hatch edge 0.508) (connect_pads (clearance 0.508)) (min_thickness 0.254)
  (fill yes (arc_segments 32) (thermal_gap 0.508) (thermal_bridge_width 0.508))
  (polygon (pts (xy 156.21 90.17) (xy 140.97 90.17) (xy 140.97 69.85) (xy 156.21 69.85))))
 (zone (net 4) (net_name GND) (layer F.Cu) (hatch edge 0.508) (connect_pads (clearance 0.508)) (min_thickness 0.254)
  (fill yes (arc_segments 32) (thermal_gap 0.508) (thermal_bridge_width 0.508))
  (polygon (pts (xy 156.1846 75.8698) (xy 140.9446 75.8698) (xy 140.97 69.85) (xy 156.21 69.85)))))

